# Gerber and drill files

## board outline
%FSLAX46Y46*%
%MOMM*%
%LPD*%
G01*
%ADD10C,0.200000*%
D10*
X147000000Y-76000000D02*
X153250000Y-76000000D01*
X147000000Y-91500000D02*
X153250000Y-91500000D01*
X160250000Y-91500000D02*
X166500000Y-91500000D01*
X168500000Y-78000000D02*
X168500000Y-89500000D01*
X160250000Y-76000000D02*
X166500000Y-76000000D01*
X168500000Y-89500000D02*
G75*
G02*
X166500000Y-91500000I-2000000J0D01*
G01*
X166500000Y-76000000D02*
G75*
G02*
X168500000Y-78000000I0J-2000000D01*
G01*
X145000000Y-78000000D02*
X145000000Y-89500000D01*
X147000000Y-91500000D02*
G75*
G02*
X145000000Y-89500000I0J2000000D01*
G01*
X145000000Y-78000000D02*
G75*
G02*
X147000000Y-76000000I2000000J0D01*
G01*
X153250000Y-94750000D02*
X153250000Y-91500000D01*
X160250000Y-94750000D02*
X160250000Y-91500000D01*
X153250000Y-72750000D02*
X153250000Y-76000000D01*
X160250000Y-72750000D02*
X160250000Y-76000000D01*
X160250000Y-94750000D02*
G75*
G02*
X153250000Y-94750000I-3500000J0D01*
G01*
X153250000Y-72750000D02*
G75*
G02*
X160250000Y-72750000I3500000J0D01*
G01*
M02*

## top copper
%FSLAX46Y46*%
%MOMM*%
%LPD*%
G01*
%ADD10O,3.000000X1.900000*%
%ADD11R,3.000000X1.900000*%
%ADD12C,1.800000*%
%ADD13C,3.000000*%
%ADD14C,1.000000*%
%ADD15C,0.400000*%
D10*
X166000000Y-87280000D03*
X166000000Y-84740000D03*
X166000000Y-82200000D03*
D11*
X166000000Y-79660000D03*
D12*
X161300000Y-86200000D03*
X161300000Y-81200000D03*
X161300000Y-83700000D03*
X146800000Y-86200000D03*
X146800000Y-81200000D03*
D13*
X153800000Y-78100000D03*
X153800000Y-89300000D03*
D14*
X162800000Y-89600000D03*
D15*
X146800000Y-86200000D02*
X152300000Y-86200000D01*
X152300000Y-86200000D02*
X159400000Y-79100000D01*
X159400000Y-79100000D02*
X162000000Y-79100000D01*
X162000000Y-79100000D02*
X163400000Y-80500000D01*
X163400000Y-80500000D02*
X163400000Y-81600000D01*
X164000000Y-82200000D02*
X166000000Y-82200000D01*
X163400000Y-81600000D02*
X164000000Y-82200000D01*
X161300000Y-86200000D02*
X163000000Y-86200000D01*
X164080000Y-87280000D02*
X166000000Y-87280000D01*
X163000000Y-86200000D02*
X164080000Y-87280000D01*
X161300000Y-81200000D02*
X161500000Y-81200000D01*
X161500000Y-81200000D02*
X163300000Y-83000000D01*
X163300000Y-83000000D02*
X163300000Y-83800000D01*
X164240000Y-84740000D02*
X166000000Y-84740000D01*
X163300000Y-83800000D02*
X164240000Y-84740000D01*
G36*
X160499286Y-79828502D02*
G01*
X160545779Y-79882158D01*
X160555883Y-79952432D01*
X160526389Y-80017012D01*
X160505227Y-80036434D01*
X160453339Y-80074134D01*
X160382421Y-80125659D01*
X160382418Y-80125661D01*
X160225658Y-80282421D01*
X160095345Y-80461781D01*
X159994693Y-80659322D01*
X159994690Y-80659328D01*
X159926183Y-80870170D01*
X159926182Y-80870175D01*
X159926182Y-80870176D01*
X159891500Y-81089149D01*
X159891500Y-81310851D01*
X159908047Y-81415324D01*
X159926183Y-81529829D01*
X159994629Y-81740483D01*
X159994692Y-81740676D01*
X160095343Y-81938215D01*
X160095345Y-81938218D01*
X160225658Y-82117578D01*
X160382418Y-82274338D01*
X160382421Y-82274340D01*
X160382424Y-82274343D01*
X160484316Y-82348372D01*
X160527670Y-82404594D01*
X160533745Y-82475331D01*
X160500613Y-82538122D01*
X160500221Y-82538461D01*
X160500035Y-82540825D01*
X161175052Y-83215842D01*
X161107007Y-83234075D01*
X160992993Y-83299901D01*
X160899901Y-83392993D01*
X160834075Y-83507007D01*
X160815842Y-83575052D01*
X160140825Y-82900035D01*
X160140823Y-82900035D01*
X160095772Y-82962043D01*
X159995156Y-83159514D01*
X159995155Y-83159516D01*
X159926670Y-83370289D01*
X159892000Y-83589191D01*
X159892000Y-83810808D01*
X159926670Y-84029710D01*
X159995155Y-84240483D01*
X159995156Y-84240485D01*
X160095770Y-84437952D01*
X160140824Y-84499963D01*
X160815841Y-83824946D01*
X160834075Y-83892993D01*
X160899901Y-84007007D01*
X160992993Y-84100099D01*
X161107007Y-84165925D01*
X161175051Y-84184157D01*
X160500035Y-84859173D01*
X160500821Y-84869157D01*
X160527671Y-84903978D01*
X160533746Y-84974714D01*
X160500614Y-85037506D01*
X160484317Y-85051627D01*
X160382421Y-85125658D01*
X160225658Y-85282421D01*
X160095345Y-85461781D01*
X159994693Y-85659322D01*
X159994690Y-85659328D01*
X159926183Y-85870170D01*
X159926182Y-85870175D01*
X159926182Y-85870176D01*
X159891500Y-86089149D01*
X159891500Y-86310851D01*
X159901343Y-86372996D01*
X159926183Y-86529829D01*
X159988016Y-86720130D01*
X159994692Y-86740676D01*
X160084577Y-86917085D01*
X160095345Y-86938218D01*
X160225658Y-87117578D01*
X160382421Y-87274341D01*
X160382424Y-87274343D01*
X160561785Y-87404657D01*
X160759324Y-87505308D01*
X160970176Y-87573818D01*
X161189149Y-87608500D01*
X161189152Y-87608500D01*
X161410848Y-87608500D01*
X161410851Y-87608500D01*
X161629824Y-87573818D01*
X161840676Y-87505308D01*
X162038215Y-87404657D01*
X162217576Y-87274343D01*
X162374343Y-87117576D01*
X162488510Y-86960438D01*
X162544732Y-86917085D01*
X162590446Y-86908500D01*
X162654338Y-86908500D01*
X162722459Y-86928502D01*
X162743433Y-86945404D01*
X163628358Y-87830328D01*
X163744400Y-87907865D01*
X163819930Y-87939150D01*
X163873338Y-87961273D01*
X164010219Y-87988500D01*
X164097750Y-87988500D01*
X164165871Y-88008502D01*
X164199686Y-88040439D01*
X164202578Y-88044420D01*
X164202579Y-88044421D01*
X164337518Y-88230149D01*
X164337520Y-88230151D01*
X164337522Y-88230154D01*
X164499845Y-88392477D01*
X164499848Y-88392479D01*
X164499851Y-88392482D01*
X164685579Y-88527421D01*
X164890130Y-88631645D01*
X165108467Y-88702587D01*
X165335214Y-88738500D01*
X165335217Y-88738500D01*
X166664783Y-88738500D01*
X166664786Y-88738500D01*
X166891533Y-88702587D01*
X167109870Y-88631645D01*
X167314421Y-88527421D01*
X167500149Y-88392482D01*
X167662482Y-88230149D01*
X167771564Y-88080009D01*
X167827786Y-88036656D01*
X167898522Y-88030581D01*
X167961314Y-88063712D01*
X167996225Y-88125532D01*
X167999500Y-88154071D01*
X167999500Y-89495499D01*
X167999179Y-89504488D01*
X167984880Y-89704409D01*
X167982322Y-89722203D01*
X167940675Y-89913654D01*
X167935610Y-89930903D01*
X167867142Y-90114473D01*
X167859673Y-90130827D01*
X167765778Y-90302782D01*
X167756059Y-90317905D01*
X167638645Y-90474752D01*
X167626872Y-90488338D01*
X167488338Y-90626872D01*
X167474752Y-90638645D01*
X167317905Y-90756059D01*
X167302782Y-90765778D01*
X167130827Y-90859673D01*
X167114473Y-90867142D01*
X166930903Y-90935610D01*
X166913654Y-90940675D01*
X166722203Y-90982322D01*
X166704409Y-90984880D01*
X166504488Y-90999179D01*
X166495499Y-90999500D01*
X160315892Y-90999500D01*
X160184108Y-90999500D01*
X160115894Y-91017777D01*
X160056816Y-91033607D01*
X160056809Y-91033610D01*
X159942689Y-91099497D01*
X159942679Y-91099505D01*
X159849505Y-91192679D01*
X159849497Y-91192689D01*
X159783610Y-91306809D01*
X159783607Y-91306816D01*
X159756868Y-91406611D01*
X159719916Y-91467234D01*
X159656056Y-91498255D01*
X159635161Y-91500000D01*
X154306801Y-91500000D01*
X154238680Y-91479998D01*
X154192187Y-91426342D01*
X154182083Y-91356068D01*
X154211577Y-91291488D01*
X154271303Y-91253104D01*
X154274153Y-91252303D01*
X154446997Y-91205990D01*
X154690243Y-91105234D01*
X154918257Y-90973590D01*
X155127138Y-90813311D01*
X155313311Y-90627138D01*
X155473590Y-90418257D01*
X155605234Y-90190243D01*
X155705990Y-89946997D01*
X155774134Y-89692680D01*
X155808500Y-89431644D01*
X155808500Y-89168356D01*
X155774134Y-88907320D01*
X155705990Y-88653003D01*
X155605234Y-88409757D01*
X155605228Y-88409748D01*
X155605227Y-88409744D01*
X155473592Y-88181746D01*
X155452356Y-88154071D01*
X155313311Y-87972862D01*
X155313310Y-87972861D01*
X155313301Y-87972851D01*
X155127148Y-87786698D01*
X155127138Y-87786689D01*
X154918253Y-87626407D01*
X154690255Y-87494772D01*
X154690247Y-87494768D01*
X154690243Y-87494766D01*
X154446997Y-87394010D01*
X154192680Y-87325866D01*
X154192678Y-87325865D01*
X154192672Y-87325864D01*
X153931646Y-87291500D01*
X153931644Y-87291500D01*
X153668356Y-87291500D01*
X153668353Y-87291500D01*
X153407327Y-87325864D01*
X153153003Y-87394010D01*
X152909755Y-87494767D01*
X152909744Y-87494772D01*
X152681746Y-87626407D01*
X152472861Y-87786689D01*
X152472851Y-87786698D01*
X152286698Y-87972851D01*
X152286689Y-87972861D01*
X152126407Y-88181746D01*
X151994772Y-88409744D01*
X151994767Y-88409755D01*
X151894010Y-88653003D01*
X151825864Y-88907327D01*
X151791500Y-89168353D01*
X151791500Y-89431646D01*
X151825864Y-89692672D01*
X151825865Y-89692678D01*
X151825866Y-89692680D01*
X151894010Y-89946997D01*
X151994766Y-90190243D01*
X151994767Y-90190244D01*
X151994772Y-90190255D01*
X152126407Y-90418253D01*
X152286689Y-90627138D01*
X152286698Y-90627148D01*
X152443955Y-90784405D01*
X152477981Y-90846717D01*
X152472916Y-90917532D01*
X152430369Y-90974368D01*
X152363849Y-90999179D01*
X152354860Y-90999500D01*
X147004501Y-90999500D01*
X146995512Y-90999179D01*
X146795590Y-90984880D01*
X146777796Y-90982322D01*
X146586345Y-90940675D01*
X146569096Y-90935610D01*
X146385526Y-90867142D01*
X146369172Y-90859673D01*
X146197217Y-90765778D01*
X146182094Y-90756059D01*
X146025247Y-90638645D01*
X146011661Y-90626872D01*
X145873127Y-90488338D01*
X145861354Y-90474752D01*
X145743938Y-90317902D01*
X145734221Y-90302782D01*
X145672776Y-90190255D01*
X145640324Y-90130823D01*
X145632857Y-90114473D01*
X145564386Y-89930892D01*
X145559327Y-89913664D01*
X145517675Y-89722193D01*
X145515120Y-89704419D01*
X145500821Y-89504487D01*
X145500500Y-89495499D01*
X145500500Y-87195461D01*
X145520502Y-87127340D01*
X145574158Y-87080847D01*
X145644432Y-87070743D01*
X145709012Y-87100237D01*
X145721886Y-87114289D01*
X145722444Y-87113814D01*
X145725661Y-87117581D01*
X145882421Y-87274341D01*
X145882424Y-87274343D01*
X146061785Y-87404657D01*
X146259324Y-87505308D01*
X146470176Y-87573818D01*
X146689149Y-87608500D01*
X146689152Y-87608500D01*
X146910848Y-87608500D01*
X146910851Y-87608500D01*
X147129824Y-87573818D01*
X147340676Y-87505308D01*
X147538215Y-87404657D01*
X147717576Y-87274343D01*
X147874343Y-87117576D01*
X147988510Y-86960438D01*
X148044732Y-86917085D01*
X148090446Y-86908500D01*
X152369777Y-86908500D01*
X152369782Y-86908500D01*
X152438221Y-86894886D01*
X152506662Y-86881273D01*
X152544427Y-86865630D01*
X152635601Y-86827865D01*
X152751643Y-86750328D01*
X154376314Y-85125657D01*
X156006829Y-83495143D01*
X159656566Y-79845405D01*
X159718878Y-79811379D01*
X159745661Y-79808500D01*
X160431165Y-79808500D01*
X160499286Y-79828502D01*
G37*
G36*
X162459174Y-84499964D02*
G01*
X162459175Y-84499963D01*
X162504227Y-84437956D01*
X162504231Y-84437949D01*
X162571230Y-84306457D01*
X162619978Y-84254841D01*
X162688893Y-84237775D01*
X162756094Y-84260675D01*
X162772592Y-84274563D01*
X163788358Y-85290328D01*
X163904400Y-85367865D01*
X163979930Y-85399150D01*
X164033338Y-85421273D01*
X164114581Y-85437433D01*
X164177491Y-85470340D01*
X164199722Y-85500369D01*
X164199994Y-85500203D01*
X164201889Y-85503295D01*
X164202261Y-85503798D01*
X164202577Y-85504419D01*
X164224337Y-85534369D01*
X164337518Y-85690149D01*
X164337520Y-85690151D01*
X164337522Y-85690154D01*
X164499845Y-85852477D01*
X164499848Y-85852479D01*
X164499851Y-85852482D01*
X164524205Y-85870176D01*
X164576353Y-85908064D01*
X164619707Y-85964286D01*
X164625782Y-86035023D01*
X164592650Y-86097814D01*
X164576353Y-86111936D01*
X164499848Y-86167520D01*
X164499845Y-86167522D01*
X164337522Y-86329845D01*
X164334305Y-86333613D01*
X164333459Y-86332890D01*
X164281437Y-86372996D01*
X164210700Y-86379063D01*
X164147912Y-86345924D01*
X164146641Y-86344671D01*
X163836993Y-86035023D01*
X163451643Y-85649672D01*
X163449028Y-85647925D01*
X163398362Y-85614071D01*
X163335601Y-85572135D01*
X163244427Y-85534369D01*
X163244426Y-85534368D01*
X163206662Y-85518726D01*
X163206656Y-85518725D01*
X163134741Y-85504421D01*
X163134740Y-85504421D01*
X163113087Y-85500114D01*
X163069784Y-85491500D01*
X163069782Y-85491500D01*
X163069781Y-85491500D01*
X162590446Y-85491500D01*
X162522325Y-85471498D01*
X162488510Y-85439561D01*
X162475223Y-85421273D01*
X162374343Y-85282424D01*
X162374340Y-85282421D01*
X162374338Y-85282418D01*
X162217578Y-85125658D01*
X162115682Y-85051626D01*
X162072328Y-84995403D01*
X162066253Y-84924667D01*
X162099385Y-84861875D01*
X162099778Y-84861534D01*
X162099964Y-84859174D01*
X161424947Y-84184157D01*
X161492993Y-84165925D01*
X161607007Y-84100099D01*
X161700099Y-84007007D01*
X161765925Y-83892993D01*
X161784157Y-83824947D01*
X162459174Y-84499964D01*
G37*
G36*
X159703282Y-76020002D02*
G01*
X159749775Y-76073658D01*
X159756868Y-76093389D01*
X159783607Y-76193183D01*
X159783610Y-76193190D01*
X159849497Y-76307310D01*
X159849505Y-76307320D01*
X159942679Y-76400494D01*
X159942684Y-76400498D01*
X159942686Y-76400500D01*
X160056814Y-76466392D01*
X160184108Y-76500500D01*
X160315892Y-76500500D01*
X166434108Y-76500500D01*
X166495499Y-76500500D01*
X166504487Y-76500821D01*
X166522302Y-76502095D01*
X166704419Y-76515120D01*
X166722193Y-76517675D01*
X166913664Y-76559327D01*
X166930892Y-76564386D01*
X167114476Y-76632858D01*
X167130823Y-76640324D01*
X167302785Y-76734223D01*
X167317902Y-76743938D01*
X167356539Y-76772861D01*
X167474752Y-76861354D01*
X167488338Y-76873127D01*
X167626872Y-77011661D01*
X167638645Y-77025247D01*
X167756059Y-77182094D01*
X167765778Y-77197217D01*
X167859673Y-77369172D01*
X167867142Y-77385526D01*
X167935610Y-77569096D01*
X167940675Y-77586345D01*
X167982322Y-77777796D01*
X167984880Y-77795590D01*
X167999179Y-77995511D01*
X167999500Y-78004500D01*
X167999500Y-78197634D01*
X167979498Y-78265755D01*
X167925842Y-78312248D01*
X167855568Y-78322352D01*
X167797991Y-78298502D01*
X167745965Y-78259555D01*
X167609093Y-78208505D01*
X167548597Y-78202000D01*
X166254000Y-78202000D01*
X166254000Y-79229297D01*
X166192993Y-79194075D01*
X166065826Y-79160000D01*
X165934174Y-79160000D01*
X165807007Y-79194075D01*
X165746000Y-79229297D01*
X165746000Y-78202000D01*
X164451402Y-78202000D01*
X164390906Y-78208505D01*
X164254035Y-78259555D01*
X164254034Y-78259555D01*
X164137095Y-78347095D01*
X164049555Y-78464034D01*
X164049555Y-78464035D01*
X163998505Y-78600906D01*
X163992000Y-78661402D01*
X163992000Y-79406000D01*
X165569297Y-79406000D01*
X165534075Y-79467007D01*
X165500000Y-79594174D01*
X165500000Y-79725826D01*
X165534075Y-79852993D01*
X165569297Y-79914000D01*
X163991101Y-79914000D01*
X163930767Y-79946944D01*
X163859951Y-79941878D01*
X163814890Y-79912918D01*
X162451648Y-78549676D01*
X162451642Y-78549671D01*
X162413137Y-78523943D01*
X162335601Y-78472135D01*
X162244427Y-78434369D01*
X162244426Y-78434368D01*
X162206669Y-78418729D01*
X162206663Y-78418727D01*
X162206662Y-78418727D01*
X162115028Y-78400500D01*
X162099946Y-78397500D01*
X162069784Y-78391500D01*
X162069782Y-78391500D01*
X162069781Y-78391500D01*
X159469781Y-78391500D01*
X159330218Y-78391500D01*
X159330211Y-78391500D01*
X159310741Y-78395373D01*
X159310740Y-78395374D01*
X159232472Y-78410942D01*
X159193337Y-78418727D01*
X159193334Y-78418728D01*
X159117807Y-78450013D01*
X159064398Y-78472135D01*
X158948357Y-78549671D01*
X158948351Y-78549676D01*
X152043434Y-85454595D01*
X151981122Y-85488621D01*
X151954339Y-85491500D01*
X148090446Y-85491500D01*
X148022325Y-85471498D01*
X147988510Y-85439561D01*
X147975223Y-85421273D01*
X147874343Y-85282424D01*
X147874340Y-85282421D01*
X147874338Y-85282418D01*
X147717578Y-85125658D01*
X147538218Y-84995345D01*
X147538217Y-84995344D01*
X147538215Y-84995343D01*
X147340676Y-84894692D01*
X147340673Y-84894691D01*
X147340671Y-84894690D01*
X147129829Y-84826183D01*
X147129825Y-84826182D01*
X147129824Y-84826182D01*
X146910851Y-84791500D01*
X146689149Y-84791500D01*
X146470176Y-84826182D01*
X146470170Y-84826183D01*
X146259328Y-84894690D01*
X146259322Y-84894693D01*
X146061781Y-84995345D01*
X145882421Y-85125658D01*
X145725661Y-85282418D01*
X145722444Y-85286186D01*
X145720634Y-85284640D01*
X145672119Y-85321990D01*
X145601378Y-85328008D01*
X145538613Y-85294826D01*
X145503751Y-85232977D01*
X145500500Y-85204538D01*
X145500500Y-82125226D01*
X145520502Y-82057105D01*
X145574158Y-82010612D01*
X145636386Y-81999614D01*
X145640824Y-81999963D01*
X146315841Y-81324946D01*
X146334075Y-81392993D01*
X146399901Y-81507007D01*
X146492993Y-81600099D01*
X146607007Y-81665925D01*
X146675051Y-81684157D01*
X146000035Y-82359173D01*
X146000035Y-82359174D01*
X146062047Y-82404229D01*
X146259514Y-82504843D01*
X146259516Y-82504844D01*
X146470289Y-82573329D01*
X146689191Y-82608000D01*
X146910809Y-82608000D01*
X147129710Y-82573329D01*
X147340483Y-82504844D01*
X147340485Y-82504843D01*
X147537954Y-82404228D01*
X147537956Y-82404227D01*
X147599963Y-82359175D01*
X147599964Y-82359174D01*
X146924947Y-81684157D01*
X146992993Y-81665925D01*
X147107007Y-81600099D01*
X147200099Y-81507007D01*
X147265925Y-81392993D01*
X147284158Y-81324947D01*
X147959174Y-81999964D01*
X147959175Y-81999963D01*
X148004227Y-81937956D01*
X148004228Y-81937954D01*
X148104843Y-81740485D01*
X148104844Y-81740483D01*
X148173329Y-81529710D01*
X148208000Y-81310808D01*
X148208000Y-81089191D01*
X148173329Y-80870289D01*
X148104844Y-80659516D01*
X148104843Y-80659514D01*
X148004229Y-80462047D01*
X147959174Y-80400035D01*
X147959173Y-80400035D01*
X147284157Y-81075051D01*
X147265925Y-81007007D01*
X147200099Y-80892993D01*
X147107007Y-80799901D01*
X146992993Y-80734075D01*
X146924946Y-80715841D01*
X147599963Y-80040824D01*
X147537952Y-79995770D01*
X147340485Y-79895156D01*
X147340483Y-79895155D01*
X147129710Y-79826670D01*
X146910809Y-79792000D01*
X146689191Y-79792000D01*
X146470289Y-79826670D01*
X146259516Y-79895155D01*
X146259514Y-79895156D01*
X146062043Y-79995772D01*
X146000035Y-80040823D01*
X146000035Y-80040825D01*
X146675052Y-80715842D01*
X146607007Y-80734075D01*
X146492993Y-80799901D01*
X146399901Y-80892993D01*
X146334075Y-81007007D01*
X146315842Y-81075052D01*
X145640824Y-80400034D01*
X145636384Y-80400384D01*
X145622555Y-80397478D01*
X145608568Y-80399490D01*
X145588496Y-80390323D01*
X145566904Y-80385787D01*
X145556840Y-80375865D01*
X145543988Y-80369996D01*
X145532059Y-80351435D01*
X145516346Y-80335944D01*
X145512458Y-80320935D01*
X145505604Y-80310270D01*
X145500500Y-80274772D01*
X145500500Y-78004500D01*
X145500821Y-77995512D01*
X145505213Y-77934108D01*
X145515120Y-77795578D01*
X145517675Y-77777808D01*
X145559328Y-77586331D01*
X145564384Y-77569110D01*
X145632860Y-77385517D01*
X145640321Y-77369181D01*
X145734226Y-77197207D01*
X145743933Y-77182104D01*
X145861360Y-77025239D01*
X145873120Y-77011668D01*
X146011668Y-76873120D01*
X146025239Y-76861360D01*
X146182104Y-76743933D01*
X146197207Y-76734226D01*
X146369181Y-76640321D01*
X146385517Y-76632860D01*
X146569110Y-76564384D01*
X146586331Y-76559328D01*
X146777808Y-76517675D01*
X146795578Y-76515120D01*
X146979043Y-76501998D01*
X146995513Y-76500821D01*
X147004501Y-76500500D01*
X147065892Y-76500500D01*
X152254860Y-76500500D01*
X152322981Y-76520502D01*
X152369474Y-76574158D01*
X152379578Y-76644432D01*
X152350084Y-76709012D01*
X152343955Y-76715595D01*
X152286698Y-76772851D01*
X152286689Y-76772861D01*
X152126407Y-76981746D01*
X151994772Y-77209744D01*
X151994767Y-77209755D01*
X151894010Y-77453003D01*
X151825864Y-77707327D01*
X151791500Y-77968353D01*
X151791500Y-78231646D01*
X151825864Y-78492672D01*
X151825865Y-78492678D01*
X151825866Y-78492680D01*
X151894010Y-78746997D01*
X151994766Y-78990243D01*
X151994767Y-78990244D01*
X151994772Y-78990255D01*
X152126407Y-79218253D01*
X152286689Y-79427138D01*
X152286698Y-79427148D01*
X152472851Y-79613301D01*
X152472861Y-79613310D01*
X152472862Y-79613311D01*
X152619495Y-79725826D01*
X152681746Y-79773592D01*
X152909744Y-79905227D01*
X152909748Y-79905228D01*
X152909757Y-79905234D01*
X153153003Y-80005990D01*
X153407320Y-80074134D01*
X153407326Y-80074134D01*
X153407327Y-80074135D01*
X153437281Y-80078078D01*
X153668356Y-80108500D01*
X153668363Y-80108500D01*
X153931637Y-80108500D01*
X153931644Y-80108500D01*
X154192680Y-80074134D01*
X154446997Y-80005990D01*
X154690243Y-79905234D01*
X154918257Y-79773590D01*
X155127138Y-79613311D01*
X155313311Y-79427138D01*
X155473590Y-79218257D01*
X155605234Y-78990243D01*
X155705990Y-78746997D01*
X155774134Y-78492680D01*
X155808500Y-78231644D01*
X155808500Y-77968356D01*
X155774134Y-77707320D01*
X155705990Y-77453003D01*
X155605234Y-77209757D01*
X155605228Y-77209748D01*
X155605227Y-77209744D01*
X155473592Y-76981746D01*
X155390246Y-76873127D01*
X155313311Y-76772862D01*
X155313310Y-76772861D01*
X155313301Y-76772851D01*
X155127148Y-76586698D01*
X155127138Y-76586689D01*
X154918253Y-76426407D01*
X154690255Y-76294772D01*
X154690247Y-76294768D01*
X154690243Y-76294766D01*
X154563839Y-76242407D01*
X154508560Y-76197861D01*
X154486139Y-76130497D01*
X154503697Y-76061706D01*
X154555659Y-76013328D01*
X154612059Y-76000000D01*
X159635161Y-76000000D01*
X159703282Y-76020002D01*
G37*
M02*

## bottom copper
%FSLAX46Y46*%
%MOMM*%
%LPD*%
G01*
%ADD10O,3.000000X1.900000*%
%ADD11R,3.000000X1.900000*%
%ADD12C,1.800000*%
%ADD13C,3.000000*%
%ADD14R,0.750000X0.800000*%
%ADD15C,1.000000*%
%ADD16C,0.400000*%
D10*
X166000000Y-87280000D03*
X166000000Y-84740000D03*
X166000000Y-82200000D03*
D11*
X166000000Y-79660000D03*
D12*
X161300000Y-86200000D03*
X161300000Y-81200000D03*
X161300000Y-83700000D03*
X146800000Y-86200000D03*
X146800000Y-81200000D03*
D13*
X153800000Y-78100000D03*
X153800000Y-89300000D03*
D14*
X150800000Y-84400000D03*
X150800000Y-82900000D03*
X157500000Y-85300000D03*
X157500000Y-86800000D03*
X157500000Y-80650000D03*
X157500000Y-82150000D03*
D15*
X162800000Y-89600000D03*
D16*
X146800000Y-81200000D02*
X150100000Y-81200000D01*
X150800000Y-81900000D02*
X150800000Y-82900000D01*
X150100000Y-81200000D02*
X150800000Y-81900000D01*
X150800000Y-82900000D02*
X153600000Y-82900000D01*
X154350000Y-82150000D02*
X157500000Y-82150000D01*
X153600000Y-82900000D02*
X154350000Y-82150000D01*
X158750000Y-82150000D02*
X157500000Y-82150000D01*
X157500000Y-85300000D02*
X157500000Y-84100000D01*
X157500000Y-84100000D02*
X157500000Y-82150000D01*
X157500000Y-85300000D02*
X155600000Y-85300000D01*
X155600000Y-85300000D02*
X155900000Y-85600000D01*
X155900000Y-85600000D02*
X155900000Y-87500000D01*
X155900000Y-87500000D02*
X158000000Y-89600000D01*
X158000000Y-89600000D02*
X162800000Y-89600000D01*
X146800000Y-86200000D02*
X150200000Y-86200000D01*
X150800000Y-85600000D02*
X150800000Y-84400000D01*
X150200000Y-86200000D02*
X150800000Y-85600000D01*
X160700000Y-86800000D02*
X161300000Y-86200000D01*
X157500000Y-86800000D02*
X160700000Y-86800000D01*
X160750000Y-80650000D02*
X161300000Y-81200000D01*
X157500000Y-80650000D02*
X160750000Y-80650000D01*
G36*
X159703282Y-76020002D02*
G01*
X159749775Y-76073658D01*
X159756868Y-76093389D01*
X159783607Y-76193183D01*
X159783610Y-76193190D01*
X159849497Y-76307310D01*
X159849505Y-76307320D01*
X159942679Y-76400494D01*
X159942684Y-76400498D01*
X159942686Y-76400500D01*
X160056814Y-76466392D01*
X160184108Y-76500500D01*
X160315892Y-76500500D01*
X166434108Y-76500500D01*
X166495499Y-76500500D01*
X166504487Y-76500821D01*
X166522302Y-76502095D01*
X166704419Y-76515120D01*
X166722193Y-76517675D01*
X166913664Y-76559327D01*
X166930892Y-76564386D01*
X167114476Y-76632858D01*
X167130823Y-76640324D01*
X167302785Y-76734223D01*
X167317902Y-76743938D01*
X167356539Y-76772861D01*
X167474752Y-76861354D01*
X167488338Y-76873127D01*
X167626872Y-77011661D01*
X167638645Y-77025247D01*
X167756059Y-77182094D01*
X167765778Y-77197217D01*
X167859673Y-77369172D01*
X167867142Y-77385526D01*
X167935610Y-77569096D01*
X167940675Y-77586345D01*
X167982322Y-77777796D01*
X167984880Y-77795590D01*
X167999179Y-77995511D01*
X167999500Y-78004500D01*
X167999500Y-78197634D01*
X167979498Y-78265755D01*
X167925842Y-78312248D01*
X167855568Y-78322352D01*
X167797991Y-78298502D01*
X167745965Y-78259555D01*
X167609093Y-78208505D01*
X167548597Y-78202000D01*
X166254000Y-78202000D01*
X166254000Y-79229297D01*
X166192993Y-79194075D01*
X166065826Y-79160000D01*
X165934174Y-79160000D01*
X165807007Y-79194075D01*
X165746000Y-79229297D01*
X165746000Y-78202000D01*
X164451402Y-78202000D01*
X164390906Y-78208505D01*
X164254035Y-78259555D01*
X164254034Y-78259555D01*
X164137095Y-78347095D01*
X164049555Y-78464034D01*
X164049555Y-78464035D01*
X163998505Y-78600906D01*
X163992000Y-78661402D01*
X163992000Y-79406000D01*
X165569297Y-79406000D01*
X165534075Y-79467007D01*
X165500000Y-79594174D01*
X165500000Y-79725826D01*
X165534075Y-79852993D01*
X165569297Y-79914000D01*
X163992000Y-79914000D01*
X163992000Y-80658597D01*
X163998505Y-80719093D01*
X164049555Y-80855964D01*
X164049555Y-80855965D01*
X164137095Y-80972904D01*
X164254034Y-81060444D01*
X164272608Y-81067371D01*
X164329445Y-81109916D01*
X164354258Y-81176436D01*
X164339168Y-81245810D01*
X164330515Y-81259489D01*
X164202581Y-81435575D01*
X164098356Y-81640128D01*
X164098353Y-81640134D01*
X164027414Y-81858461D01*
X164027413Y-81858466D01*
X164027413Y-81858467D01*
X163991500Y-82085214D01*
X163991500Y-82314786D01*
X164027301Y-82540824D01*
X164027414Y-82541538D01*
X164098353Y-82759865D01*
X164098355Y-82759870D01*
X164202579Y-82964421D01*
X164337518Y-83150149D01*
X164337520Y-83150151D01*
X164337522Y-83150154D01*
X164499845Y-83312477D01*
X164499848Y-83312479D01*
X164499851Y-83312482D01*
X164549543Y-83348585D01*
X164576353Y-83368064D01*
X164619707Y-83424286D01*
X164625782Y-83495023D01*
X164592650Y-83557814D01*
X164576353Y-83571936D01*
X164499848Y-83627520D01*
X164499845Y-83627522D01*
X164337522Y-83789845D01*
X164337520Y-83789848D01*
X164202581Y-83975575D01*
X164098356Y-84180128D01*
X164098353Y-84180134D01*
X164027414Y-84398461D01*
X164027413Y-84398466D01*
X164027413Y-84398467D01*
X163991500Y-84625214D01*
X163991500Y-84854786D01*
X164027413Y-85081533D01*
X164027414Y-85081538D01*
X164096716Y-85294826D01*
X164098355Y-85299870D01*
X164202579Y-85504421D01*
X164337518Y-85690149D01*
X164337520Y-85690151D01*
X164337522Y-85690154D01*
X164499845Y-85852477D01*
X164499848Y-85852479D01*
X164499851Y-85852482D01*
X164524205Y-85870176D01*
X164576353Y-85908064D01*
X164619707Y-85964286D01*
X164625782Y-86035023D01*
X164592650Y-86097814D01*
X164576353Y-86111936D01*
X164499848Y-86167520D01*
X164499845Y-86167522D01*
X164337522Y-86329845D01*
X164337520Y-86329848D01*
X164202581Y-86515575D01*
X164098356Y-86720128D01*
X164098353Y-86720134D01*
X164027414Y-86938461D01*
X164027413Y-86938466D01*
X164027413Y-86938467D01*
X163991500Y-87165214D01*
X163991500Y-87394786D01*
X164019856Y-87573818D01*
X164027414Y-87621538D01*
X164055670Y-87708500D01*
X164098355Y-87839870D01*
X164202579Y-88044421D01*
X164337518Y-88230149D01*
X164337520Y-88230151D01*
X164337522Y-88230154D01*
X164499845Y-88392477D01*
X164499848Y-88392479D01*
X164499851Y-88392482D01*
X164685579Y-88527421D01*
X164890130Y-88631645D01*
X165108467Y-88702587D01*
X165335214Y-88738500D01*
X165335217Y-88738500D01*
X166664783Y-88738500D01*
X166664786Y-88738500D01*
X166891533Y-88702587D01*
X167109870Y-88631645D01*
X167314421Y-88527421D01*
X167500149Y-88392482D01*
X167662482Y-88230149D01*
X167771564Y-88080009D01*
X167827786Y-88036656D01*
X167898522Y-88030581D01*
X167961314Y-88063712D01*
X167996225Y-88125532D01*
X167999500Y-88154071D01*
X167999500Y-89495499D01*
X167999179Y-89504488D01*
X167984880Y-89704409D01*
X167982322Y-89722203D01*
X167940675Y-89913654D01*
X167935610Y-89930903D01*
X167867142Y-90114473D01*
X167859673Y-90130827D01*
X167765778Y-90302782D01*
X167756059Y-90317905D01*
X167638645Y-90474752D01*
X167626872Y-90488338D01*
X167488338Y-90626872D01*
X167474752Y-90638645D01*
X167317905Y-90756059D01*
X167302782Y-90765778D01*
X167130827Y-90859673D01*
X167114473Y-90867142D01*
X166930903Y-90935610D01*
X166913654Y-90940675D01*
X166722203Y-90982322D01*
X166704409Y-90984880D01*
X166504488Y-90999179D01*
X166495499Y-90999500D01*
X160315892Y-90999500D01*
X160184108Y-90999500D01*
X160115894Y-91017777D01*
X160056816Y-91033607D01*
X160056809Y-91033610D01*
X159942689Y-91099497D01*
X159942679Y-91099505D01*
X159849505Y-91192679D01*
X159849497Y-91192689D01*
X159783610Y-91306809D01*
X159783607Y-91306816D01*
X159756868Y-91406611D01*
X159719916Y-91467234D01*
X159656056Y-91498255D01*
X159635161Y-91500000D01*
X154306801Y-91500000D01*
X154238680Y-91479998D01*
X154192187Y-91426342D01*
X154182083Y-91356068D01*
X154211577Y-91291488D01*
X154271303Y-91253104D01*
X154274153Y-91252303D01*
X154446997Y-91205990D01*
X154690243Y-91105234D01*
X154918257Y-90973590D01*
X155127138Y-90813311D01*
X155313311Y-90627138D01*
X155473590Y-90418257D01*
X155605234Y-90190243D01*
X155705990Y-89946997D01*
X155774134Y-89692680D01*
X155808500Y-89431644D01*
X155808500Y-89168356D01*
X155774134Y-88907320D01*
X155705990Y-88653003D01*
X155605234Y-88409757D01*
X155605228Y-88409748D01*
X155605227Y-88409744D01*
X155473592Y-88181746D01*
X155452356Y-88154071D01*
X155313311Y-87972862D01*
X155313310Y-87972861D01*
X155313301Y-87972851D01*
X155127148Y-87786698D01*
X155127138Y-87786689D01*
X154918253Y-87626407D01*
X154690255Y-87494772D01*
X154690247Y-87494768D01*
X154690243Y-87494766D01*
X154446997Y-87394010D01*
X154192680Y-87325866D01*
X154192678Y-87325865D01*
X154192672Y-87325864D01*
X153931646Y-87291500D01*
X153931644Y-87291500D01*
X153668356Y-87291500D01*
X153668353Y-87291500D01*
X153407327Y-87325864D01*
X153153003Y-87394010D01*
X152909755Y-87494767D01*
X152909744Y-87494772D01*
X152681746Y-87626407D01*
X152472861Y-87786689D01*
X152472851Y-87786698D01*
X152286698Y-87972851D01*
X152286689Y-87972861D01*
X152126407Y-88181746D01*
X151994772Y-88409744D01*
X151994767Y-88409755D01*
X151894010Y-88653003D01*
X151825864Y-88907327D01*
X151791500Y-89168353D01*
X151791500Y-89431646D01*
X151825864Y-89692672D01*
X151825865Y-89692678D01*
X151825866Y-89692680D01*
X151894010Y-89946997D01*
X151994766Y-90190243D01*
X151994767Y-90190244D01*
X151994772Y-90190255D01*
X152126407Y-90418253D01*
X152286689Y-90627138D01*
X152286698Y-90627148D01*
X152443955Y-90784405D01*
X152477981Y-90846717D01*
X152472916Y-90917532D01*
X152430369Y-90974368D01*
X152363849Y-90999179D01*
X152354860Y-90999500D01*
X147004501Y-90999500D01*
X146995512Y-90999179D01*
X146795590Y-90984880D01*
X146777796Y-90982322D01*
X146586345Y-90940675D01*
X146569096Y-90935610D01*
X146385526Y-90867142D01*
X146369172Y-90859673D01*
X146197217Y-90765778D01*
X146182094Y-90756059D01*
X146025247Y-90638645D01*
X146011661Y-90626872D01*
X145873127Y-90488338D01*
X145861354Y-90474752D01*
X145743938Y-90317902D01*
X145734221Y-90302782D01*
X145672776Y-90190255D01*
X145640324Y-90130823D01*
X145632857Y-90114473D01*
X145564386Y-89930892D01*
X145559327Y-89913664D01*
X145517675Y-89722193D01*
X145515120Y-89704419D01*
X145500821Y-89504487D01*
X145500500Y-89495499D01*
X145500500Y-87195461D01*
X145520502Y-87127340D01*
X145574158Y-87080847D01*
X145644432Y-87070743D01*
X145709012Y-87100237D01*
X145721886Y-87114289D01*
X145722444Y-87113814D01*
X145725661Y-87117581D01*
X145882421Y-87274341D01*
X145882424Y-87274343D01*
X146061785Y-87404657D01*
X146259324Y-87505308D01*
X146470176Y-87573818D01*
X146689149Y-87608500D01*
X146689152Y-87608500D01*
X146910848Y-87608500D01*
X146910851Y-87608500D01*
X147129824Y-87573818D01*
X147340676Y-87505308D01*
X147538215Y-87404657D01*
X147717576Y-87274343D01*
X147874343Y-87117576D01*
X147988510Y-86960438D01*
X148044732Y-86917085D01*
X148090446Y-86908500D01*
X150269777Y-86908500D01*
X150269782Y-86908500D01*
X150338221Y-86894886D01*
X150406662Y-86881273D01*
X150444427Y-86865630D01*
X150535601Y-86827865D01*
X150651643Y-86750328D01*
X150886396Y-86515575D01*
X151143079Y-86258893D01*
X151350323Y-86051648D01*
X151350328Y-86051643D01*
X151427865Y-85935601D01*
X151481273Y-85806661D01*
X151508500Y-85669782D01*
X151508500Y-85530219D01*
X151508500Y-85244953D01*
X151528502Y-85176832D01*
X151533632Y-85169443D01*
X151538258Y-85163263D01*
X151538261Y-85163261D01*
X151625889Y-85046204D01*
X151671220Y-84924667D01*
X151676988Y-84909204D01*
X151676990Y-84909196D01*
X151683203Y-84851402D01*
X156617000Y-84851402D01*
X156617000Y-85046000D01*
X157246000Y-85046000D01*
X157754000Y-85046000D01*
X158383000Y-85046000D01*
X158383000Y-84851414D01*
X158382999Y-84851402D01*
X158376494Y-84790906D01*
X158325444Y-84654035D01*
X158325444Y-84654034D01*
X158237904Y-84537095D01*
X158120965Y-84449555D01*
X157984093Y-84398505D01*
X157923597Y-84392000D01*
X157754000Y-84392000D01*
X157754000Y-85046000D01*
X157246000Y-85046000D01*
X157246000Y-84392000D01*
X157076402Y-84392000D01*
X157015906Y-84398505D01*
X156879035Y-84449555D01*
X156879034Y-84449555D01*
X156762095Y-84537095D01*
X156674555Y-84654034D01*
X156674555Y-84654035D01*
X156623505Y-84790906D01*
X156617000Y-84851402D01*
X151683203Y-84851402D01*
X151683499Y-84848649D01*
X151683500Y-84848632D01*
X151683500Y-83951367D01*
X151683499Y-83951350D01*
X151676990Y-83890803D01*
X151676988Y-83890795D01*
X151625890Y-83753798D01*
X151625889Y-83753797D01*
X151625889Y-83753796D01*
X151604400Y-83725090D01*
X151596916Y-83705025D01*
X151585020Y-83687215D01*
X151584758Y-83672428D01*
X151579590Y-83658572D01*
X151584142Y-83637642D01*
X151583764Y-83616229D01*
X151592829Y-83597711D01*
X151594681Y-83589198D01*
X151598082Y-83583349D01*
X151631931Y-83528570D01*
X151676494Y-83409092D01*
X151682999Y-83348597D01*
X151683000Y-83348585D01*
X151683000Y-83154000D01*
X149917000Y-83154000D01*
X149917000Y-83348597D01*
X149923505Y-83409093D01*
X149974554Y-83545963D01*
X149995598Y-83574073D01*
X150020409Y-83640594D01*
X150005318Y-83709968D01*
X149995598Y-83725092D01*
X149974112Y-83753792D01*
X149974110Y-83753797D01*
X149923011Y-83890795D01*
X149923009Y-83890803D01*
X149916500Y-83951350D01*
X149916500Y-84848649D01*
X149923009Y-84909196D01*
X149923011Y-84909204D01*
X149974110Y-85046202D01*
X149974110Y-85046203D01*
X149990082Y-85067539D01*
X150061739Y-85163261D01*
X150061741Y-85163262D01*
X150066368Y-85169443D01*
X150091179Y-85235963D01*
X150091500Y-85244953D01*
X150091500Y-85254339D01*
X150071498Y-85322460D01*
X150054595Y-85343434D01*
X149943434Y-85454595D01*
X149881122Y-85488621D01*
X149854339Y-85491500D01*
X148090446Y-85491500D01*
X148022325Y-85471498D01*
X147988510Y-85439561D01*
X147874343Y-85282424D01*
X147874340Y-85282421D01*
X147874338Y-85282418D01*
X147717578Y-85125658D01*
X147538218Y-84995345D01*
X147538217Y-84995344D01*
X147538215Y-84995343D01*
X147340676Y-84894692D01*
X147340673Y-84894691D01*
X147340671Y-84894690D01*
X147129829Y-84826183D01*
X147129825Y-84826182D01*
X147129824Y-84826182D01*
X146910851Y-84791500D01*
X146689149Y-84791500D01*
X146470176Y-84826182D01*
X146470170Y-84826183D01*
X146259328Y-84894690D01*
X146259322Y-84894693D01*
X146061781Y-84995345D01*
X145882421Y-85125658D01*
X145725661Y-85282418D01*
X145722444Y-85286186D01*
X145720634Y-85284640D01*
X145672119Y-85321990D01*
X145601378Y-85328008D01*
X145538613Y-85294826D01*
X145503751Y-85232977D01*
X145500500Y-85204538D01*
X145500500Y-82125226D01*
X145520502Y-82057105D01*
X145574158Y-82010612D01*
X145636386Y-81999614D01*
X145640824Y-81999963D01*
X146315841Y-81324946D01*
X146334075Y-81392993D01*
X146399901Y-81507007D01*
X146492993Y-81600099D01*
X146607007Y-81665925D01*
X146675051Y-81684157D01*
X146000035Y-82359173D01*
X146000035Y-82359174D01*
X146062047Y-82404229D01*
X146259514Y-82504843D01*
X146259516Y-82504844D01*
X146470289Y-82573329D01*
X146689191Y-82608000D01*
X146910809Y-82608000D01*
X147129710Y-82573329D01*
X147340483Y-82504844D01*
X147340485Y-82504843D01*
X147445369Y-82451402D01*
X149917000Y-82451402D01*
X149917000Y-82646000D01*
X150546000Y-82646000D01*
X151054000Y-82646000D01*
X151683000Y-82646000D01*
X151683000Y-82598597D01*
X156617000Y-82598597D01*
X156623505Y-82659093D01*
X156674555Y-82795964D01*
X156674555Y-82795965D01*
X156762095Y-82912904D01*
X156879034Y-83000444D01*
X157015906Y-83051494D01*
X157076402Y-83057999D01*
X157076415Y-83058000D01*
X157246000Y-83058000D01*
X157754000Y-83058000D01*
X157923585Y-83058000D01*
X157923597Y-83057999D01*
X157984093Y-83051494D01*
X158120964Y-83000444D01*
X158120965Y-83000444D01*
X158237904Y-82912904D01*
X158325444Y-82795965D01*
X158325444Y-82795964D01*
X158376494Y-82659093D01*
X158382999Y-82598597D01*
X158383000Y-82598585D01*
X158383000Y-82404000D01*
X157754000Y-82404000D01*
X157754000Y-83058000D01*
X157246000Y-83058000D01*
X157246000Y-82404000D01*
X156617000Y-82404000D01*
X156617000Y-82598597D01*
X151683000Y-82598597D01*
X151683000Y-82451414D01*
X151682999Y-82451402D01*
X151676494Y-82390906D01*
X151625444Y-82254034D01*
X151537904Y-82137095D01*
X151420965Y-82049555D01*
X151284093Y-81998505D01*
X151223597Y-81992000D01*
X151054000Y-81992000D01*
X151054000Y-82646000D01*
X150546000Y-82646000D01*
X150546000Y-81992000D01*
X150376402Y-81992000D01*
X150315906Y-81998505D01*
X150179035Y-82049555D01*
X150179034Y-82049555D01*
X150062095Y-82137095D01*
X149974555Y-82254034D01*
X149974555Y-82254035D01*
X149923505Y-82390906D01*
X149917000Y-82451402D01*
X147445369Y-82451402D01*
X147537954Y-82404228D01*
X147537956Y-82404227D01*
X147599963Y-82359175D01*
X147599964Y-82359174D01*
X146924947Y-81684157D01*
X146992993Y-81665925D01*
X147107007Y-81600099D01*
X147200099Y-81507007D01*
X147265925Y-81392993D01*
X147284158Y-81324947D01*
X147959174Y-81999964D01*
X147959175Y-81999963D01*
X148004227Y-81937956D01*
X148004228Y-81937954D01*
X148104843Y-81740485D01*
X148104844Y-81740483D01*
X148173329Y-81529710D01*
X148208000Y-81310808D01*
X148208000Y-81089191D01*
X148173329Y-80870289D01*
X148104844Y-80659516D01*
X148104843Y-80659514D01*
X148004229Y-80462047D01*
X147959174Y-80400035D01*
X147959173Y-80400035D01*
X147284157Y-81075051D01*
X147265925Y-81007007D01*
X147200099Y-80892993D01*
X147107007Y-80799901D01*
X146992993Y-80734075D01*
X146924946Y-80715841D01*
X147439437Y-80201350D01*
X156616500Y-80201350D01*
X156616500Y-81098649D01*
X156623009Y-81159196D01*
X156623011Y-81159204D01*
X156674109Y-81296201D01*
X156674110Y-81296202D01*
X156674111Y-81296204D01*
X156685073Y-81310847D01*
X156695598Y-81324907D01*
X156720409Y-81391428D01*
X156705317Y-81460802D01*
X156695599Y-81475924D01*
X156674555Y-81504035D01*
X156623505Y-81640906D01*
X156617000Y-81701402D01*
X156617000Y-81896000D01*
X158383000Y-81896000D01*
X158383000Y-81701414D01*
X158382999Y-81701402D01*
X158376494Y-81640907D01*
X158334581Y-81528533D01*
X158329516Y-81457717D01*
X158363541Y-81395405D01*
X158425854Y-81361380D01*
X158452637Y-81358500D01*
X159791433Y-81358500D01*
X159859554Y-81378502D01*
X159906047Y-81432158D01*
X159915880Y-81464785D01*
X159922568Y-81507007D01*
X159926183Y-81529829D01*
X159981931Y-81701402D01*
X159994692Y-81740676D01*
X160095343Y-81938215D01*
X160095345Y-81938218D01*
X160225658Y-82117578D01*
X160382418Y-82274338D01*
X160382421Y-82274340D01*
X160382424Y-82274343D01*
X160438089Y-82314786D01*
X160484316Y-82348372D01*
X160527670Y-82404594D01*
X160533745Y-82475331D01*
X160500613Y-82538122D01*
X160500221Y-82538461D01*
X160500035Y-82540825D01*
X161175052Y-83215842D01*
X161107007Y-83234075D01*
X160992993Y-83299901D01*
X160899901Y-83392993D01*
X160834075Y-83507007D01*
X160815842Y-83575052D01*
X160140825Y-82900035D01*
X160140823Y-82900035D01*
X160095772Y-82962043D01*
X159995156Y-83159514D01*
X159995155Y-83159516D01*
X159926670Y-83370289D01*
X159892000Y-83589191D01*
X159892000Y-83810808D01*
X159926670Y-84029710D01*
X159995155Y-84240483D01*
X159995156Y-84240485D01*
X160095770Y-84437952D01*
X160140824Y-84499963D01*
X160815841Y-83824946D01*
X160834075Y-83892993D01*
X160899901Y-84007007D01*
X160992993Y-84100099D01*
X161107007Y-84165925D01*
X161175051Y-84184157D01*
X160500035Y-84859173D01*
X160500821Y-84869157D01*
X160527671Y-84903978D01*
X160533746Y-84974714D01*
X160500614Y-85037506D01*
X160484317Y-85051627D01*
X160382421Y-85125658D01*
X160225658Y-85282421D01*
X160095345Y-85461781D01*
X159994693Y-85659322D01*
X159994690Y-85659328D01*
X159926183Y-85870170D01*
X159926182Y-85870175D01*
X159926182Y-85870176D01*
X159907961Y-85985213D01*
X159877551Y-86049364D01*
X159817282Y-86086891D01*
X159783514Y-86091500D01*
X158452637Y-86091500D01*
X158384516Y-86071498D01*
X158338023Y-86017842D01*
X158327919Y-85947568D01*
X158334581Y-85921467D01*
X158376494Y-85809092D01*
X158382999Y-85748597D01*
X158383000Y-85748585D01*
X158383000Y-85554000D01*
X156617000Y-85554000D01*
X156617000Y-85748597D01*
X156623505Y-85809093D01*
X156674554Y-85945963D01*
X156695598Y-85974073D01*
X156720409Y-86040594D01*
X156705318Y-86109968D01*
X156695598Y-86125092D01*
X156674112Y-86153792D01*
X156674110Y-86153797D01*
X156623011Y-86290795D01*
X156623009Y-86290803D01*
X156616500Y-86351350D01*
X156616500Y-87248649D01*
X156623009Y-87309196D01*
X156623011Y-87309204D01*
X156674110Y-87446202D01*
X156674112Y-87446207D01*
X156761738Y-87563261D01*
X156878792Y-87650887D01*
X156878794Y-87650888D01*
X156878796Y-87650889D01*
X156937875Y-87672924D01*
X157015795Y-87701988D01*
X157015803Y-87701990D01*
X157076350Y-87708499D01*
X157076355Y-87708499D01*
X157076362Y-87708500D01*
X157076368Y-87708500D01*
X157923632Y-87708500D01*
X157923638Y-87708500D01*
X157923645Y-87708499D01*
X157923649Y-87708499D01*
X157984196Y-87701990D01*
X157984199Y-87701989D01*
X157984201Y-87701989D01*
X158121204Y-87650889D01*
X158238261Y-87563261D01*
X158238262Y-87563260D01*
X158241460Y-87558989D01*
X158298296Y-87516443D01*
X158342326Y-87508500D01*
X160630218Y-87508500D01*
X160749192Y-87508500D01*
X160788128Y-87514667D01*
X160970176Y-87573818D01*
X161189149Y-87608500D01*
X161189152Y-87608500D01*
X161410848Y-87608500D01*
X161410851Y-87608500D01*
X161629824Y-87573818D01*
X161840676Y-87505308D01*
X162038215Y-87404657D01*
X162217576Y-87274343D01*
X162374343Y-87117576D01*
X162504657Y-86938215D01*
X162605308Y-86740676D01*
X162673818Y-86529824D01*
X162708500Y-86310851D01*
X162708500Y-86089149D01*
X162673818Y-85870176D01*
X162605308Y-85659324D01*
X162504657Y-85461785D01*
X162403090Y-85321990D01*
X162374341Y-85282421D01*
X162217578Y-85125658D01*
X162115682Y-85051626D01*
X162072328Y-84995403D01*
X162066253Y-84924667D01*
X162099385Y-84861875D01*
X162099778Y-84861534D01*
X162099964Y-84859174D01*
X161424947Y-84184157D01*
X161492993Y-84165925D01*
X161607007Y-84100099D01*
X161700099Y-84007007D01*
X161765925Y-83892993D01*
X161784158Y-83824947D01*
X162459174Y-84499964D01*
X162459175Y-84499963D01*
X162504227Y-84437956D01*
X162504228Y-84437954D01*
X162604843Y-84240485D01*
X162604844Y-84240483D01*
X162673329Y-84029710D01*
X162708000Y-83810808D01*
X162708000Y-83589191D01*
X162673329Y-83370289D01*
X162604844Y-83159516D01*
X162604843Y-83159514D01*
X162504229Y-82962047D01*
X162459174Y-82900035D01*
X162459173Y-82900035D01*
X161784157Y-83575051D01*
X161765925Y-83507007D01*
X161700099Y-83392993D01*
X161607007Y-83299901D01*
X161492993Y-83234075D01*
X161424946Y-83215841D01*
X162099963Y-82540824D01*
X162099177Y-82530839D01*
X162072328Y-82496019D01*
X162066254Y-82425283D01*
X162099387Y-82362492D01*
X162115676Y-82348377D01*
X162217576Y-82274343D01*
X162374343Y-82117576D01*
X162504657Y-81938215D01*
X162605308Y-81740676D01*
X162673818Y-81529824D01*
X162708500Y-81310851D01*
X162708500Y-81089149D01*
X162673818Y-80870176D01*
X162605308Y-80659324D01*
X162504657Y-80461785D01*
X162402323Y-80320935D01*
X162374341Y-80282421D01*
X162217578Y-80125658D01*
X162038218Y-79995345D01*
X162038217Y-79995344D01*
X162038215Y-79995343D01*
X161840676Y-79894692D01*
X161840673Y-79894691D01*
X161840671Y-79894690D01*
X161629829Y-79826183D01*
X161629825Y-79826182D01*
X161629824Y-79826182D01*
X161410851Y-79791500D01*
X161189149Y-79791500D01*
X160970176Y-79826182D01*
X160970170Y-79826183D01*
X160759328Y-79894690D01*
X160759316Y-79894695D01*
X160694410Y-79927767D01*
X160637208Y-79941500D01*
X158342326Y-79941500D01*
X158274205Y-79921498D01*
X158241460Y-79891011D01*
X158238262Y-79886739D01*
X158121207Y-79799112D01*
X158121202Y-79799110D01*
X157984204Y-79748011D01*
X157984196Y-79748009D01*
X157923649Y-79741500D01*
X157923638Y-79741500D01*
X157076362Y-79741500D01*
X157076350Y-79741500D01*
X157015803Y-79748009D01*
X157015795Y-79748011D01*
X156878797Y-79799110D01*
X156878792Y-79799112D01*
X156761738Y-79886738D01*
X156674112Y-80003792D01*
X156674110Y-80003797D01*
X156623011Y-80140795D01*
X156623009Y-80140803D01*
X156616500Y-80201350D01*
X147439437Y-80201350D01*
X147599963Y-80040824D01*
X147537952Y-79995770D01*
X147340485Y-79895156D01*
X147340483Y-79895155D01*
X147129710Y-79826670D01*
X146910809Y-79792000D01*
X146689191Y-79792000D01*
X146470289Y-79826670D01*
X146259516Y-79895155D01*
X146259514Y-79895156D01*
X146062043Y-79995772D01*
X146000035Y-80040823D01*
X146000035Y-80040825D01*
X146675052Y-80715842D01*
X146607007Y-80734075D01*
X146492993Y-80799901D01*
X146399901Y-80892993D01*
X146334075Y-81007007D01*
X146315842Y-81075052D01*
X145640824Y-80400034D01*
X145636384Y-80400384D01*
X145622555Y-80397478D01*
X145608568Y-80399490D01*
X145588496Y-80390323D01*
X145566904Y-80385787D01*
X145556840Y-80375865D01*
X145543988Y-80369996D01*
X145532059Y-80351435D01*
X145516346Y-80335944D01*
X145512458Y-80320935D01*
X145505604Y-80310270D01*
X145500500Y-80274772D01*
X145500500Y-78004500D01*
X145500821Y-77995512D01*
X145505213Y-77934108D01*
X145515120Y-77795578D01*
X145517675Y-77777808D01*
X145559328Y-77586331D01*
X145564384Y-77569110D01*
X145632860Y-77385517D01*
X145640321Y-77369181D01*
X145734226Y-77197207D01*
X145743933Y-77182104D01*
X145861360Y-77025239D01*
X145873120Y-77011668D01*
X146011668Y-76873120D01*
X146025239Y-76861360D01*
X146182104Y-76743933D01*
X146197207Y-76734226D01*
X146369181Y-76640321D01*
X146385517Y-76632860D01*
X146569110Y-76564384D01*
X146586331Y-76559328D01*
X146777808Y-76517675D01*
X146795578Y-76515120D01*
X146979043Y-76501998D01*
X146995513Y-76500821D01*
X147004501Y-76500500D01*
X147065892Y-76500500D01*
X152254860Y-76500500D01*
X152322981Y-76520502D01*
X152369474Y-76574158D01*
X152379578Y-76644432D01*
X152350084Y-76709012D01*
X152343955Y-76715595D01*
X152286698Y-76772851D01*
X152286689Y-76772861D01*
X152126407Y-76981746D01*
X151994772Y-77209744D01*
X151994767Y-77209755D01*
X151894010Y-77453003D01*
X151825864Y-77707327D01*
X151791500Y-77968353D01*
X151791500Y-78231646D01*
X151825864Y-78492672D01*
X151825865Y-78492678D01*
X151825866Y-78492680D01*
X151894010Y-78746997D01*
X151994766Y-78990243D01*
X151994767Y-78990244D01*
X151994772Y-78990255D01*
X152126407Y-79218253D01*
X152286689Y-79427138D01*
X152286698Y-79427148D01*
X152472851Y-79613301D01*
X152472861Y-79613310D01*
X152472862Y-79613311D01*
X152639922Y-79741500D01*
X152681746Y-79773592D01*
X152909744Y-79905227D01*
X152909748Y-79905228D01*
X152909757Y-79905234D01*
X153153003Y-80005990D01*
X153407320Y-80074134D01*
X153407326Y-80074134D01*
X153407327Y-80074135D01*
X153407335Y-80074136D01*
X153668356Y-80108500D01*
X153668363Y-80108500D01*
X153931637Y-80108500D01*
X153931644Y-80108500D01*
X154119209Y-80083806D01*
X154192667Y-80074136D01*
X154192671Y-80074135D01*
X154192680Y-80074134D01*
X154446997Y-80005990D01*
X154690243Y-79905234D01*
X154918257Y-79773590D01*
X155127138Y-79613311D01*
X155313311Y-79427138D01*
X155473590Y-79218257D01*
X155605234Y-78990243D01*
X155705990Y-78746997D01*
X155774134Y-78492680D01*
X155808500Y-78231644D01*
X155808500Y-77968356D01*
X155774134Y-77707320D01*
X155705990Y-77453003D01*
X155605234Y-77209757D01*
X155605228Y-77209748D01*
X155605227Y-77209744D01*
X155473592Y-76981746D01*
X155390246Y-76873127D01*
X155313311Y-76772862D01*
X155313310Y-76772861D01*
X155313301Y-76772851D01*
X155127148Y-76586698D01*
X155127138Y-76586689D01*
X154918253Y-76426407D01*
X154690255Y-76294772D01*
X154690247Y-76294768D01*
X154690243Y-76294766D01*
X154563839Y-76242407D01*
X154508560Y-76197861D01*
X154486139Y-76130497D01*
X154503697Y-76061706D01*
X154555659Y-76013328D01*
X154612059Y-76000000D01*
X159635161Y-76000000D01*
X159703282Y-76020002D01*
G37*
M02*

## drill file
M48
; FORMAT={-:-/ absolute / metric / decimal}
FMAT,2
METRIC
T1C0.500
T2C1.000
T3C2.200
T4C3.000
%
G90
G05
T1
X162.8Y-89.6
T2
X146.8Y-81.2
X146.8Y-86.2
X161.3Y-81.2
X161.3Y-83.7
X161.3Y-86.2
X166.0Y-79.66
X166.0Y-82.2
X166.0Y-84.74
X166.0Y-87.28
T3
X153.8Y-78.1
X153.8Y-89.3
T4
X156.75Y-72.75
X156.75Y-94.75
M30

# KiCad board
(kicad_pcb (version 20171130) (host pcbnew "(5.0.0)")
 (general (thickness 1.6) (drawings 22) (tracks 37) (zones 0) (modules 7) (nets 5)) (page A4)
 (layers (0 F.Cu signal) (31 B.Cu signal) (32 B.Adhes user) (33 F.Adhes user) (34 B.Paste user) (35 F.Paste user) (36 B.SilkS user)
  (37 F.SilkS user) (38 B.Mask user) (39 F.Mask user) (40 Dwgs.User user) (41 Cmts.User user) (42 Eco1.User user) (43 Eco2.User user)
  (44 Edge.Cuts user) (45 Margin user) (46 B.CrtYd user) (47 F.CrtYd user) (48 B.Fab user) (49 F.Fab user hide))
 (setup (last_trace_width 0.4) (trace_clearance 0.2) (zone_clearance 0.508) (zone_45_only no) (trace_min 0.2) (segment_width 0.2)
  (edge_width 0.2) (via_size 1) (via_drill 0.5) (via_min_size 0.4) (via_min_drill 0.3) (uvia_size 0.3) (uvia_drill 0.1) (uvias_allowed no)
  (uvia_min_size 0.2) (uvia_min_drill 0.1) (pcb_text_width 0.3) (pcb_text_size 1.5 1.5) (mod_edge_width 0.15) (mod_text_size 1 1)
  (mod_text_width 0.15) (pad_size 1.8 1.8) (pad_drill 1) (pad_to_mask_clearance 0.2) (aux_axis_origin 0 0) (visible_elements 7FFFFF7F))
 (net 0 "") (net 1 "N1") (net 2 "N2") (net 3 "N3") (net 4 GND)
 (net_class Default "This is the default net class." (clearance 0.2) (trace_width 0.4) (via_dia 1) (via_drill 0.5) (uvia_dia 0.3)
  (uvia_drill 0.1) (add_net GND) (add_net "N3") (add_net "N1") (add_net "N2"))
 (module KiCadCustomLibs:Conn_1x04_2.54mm (layer F.Cu) (at 166 79.66)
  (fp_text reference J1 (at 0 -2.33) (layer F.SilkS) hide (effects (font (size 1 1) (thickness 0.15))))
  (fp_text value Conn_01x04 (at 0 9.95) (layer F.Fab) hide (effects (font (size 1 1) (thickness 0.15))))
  (pad 4 thru_hole oval (at 0 7.62) (size 3 1.9) (drill 1) (layers *.Cu *.Mask) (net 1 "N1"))
  (pad 3 thru_hole oval (at 0 5.08) (size 3 1.9) (drill 1) (layers *.Cu *.Mask) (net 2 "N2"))
  (pad 2 thru_hole oval (at 0 2.54) (size 3 1.9) (drill 1) (layers *.Cu *.Mask) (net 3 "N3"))
  (pad 1 thru_hole rect (at 0 0) (size 3 1.9) (drill 1) (layers *.Cu *.Mask) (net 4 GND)))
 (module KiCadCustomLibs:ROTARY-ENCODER (layer F.Cu) (at 153.8 83.7 90)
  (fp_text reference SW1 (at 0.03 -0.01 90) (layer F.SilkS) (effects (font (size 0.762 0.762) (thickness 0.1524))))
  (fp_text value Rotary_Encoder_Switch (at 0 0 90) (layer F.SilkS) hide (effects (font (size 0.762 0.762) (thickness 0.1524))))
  (pad 1 thru_hole circle (at -2.5 7.5 90) (size 1.8 1.8) (drill 1) (layers *.Cu *.Mask F.SilkS) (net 1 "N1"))
  (pad 3 thru_hole circle (at 2.5 7.5 90) (size 1.8 1.8) (drill 1) (layers *.Cu *.Mask F.SilkS) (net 2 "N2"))
  (pad 2 thru_hole circle (at 0 7.5 90) (size 1.8 1.8) (drill 1) (layers *.Cu *.Mask F.SilkS) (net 4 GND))
  (pad 4 thru_hole circle (at -2.5 -7 90) (size 1.8 1.8) (drill 1) (layers *.Cu *.Mask F.SilkS) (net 3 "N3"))
  (pad 5 thru_hole circle (at 2.5 -7 90) (size 1.8 1.8) (drill 1) (layers *.Cu *.Mask F.SilkS) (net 4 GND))
  (pad "" thru_hole circle (at 5.6 0 90) (size 3 3) (drill 2.2) (layers *.Cu *.Mask F.SilkS))
  (pad "" thru_hole circle (at -5.6 0 90) (size 3 3) (drill 2.2) (layers *.Cu *.Mask F.SilkS)))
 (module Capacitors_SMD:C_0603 (layer B.Cu) (at 150.8 83.65 90)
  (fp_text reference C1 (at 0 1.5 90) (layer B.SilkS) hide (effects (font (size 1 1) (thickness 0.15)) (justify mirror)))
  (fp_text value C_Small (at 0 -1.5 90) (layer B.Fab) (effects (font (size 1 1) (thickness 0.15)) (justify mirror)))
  (pad 1 smd rect (at -0.75 0 90) (size 0.8 0.75) (layers B.Cu B.Paste B.Mask) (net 3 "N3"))
  (pad 2 smd rect (at 0.75 0 90) (size 0.8 0.75) (layers B.Cu B.Paste B.Mask) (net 4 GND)))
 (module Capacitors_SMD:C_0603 (layer B.Cu) (at 157.5 86.05 90)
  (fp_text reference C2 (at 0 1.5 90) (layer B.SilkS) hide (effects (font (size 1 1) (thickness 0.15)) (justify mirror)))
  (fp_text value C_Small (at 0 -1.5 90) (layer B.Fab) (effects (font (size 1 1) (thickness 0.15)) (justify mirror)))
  (pad 2 smd rect (at 0.75 0 90) (size 0.8 0.75) (layers B.Cu B.Paste B.Mask) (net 4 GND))
  (pad 1 smd rect (at -0.75 0 90) (size 0.8 0.75) (layers B.Cu B.Paste B.Mask) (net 1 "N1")))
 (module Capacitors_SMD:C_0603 (layer B.Cu) (at 157.5 81.4 270)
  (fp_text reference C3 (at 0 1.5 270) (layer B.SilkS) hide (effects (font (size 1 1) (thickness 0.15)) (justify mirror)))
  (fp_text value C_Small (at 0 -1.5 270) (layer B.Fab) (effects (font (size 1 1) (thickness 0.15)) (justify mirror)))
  (pad 1 smd rect (at -0.75 0 270) (size 0.8 0.75) (layers B.Cu B.Paste B.Mask) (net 2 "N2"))
  (pad 2 smd rect (at 0.75 0 270) (size 0.8 0.75) (layers B.Cu B.Paste B.Mask) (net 4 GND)))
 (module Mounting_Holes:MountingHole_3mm (layer F.Cu) (at 156.75 72.75)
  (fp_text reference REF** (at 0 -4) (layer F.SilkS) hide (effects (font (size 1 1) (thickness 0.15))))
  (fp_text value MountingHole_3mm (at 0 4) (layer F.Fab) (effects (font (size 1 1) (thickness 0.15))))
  (pad 1 np_thru_hole circle (at 0 0) (size 3 3) (drill 3) (layers *.Cu *.Mask)))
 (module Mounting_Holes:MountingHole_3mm (layer F.Cu) (at 156.75 94.75)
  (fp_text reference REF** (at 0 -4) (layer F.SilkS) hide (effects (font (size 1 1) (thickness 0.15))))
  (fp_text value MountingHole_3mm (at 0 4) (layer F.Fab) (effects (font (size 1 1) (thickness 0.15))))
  (pad 1 np_thru_hole circle (at 0 0) (size 3 3) (drill 3) (layers *.Cu *.Mask)))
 (gr_line (start 147 76) (end 153.25 76) (layer Edge.Cuts) (width 0.2))
 (gr_line (start 147 91.5) (end 153.25 91.5) (layer Edge.Cuts) (width 0.2))
 (gr_line (start 160.25 91.5) (end 166.5 91.5) (layer Edge.Cuts) (width 0.2))
 (gr_line (start 168.5 78) (end 168.5 89.5) (layer Edge.Cuts) (width 0.2))
 (gr_line (start 160.25 76) (end 166.5 76) (layer Edge.Cuts) (width 0.2))
 (gr_arc (start 166.5 89.5) (end 166.5 91.5) (angle -90) (layer Edge.Cuts) (width 0.2))
 (gr_arc (start 166.5 78) (end 168.5 78) (angle -90) (layer Edge.Cuts) (width 0.2))
 (gr_line (start 145 78) (end 145 89.5) (layer Edge.Cuts) (width 0.2))
 (gr_arc (start 147 89.5) (end 145 89.5) (angle -90) (layer Edge.Cuts) (width 0.2))
 (gr_arc (start 147 78) (end 147 76) (angle -90) (layer Edge.Cuts) (width 0.2))
 (gr_line (start 153.25 94.75) (end 153.25 91.5) (layer Edge.Cuts) (width 0.2))
 (gr_line (start 160.25 94.75) (end 160.25 91.5) (layer Edge.Cuts) (width 0.2))
 (gr_line (start 153.25 72.75) (end 153.25 76) (layer Edge.Cuts) (width 0.2))
 (gr_line (start 160.25 72.75) (end 160.25 76) (layer Edge.Cuts) (width 0.2))
 (gr_arc (start 156.75 94.75) (end 153.25 94.75) (angle -180) (layer Edge.Cuts) (width 0.2))
 (gr_arc (start 156.75 72.75) (end 160.25 72.75) (angle -180) (layer Edge.Cuts) (width 0.2))
 (segment (start 146.8 81.2) (end 150.1 81.2) (width 0.4) (layer B.Cu) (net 4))
 (segment (start 150.8 81.9) (end 150.8 82.9) (width 0.4) (layer B.Cu) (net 4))
 (segment (start 150.1 81.2) (end 150.8 81.9) (width 0.4) (layer B.Cu) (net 4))
 (segment (start 150.8 82.9) (end 153.6 82.9) (width 0.4) (layer B.Cu) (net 4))
 (segment (start 154.35 82.15) (end 157.5 82.15) (width 0.4) (layer B.Cu) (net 4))
 (segment (start 153.6 82.9) (end 154.35 82.15) (width 0.4) (layer B.Cu) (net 4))
 (segment (start 158.75 82.15) (end 157.5 82.15) (width 0.4) (layer B.Cu) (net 4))
 (segment (start 157.5 85.3) (end 157.5 84.1) (width 0.4) (layer B.Cu) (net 4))
 (segment (start 157.5 84.1) (end 157.5 82.15) (width 0.4) (layer B.Cu) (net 4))
 (segment (start 157.5 85.3) (end 155.6 85.3) (width 0.4) (layer B.Cu) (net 4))
 (segment (start 155.6 85.3) (end 155.9 85.6) (width 0.4) (layer B.Cu) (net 4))
 (segment (start 155.9 85.6) (end 155.9 87.5) (width 0.4) (layer B.Cu) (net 4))
 (via (at 162.8 89.6) (size 1) (drill 0.5) (layers F.Cu B.Cu) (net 4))
 (segment (start 155.9 87.5) (end 158 89.6) (width 0.4) (layer B.Cu) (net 4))
 (segment (start 158 89.6) (end 162.8 89.6) (width 0.4) (layer B.Cu) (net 4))
 (segment (start 146.8 86.2) (end 150.2 86.2) (width 0.4) (layer B.Cu) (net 3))
 (segment (start 150.8 85.6) (end 150.8 84.4) (width 0.4) (layer B.Cu) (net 3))
 (segment (start 150.2 86.2) (end 150.8 85.6) (width 0.4) (layer B.Cu) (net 3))
 (segment (start 146.8 86.2) (end 152.3 86.2) (width 0.4) (layer F.Cu) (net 3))
 (segment (start 152.3 86.2) (end 159.4 79.1) (width 0.4) (layer F.Cu) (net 3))
 (segment (start 159.4 79.1) (end 162 79.1) (width 0.4) (layer F.Cu) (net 3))
 (segment (start 162 79.1) (end 163.4 80.5) (width 0.4) (layer F.Cu) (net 3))
 (segment (start 163.4 80.5) (end 163.4 81.6) (width 0.4) (layer F.Cu) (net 3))
 (segment (start 164 82.2) (end 166 82.2) (width 0.4) (layer F.Cu) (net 3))
 (segment (start 163.4 81.6) (end 164 82.2) (width 0.4) (layer F.Cu) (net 3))
 (segment (start 161.3 86.2) (end 163 86.2) (width 0.4) (layer F.Cu) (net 1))
 (segment (start 164.08 87.28) (end 166 87.28) (width 0.4) (layer F.Cu) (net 1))
 (segment (start 163 86.2) (end 164.08 87.28) (width 0.4) (layer F.Cu) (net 1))
 (segment (start 160.7 86.8) (end 161.3 86.2) (width 0.4) (layer B.Cu) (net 1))
 (segment (start 157.5 86.8) (end 160.7 86.8) (width 0.4) (layer B.Cu) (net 1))
 (segment (start 161.3 81.2) (end 161.5 81.2) (width 0.4) (layer F.Cu) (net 2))
 (segment (start 161.5 81.2) (end 163.3 83) (width 0.4) (layer F.Cu) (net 2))
 (segment (start 163.3 83) (end 163.3 83.8) (width 0.4) (layer F.Cu) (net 2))
 (segment (start 164.24 84.74) (end 166 84.74) (width 0.4) (layer F.Cu) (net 2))
 (segment (start 163.3 83.8) (end 164.24 84.74) (width 0.4) (layer F.Cu) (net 2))
 (segment (start 160.75 80.65) (end 161.3 81.2) (width 0.4) (layer B.Cu) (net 2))
 (segment (start 157.5 80.65) (end 160.75 80.65) (width 0.4) (layer B.Cu) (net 2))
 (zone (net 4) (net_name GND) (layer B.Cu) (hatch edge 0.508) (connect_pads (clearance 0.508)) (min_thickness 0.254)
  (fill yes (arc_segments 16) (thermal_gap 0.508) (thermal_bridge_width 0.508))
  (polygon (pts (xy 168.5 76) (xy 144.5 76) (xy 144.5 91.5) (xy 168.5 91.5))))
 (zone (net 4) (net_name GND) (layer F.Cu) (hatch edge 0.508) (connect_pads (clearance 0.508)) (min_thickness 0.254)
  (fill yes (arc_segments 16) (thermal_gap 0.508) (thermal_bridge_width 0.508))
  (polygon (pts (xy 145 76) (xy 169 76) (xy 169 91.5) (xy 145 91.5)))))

